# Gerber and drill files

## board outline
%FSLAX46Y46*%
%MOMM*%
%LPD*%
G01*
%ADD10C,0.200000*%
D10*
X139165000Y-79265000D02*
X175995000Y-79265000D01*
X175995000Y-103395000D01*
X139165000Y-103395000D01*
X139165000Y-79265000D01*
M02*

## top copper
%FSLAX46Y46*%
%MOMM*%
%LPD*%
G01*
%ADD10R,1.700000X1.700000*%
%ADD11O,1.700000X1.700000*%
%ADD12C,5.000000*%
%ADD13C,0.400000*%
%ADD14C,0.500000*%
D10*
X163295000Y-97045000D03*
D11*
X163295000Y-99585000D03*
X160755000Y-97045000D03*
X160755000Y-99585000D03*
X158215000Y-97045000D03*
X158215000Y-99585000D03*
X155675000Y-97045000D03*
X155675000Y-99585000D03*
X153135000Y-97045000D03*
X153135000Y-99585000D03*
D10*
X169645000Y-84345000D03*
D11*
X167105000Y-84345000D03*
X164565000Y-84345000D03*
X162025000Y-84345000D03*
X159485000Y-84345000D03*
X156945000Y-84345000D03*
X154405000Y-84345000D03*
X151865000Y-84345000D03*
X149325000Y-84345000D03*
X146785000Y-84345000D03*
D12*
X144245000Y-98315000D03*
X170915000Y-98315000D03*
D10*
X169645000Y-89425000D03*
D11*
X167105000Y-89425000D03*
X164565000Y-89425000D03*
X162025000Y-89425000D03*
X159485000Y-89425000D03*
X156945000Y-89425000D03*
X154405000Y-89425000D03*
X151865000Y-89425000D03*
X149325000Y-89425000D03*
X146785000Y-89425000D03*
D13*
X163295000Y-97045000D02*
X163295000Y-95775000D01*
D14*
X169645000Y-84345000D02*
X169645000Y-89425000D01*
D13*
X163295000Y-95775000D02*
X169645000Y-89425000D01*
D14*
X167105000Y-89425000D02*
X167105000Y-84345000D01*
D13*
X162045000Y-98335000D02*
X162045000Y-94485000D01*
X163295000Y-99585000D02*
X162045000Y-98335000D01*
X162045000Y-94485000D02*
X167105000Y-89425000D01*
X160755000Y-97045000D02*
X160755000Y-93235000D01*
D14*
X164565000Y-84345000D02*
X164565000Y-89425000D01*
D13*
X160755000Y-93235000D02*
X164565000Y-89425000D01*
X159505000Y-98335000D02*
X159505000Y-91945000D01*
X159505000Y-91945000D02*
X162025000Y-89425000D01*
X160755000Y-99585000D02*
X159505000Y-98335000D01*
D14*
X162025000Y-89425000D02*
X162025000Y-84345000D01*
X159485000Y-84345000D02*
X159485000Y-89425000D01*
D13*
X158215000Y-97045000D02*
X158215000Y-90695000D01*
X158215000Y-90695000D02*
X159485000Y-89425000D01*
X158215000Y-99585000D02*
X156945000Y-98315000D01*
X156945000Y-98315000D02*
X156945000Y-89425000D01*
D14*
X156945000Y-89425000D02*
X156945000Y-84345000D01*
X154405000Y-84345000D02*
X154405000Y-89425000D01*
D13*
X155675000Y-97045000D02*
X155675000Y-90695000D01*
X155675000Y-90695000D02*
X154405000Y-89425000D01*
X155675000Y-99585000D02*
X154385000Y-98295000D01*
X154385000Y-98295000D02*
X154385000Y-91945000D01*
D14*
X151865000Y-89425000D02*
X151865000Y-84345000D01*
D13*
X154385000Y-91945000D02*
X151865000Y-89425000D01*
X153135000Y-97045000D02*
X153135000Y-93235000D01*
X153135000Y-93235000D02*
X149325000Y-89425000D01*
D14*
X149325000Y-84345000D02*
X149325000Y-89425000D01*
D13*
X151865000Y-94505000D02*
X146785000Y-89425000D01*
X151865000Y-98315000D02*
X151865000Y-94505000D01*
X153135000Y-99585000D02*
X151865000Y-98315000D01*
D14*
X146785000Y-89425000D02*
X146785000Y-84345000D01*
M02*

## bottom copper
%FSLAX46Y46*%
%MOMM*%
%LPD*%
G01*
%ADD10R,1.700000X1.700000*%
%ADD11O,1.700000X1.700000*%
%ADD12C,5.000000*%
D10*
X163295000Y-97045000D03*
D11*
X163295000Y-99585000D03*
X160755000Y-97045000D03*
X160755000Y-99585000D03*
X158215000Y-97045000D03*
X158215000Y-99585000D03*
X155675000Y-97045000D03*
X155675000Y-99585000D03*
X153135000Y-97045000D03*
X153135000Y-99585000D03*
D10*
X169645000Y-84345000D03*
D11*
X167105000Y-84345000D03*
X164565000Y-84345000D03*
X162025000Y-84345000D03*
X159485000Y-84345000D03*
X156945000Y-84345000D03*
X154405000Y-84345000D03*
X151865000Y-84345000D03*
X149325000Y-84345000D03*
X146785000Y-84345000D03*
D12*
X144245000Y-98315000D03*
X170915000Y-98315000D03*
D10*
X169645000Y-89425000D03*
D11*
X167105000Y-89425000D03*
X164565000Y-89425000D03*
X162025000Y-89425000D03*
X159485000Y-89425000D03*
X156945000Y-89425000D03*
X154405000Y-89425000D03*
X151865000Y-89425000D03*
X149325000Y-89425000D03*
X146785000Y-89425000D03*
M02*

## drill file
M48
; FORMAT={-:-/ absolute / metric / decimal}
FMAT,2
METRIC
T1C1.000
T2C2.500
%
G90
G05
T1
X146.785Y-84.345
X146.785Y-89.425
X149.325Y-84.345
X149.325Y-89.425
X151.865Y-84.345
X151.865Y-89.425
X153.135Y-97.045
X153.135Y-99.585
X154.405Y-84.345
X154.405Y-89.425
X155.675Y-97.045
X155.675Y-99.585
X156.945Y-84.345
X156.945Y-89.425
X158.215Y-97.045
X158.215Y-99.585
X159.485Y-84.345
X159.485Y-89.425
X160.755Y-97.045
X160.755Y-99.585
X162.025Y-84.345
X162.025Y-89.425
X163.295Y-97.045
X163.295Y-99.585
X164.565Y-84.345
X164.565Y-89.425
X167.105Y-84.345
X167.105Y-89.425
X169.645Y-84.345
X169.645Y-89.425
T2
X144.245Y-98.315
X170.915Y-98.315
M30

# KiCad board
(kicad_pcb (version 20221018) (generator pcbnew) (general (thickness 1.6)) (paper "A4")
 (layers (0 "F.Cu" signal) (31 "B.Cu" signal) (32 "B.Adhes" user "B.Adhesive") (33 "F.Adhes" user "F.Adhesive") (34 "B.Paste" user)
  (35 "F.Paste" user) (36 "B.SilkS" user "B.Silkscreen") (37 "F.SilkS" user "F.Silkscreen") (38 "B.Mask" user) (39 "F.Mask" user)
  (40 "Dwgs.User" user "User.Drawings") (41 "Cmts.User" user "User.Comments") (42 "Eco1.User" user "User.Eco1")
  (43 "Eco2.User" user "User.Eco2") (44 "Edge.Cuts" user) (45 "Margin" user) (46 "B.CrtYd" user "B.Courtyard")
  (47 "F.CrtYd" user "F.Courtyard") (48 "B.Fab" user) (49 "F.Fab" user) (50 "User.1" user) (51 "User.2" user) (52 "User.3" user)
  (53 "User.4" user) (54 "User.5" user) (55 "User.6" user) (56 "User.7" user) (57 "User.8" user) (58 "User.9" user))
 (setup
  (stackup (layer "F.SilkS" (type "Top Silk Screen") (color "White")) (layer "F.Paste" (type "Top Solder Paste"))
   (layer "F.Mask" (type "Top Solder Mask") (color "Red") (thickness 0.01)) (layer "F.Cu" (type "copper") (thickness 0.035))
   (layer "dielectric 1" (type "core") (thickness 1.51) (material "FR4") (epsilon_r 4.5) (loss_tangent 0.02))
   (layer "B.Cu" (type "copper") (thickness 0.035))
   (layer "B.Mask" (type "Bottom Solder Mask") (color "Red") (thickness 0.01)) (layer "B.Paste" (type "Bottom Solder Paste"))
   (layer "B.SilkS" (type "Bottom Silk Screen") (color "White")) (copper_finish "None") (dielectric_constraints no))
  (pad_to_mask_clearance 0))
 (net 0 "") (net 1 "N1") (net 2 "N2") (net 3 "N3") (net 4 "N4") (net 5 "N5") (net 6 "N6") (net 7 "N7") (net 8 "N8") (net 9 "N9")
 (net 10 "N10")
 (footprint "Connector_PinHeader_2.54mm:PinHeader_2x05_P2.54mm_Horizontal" (layer "F.Cu") (at 163.295 97.045 -90)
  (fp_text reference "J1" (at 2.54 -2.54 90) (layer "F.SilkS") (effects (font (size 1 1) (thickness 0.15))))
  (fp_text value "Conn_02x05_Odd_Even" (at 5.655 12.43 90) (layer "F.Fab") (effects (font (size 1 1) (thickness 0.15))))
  (pad "1" thru_hole rect (at 0 0 270) (size 1.7 1.7) (drill 1) (layers "*.Cu" "*.Mask") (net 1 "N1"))
  (pad "2" thru_hole oval (at 2.54 0 270) (size 1.7 1.7) (drill 1) (layers "*.Cu" "*.Mask") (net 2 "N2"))
  (pad "3" thru_hole oval (at 0 2.54 270) (size 1.7 1.7) (drill 1) (layers "*.Cu" "*.Mask") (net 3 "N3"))
  (pad "4" thru_hole oval (at 2.54 2.54 270) (size 1.7 1.7) (drill 1) (layers "*.Cu" "*.Mask") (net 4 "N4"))
  (pad "5" thru_hole oval (at 0 5.08 270) (size 1.7 1.7) (drill 1) (layers "*.Cu" "*.Mask") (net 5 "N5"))
  (pad "6" thru_hole oval (at 2.54 5.08 270) (size 1.7 1.7) (drill 1) (layers "*.Cu" "*.Mask") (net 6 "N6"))
  (pad "7" thru_hole oval (at 0 7.62 270) (size 1.7 1.7) (drill 1) (layers "*.Cu" "*.Mask") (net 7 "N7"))
  (pad "8" thru_hole oval (at 2.54 7.62 270) (size 1.7 1.7) (drill 1) (layers "*.Cu" "*.Mask") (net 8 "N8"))
  (pad "9" thru_hole oval (at 0 10.16 270) (size 1.7 1.7) (drill 1) (layers "*.Cu" "*.Mask") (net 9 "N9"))
  (pad "10" thru_hole oval (at 2.54 10.16 270) (size 1.7 1.7) (drill 1) (layers "*.Cu" "*.Mask") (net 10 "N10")))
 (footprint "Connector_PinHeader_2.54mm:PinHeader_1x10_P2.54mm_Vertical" (layer "F.Cu") (at 169.645 84.345 -90)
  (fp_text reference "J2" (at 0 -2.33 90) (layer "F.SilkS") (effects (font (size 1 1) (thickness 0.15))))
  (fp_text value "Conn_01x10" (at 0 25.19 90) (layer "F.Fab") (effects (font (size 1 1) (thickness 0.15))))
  (pad "1" thru_hole rect (at 0 0 270) (size 1.7 1.7) (drill 1) (layers "*.Cu" "*.Mask") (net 1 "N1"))
  (pad "2" thru_hole oval (at 0 2.54 270) (size 1.7 1.7) (drill 1) (layers "*.Cu" "*.Mask") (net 2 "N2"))
  (pad "3" thru_hole oval (at 0 5.08 270) (size 1.7 1.7) (drill 1) (layers "*.Cu" "*.Mask") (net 3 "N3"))
  (pad "4" thru_hole oval (at 0 7.62 270) (size 1.7 1.7) (drill 1) (layers "*.Cu" "*.Mask") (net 4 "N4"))
  (pad "5" thru_hole oval (at 0 10.16 270) (size 1.7 1.7) (drill 1) (layers "*.Cu" "*.Mask") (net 5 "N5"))
  (pad "6" thru_hole oval (at 0 12.7 270) (size 1.7 1.7) (drill 1) (layers "*.Cu" "*.Mask") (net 6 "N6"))
  (pad "7" thru_hole oval (at 0 15.24 270) (size 1.7 1.7) (drill 1) (layers "*.Cu" "*.Mask") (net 7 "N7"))
  (pad "8" thru_hole oval (at 0 17.78 270) (size 1.7 1.7) (drill 1) (layers "*.Cu" "*.Mask") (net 8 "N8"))
  (pad "9" thru_hole oval (at 0 20.32 270) (size 1.7 1.7) (drill 1) (layers "*.Cu" "*.Mask") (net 9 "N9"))
  (pad "10" thru_hole oval (at 0 22.86 270) (size 1.7 1.7) (drill 1) (layers "*.Cu" "*.Mask") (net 10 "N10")))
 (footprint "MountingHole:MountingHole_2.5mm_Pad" (layer "F.Cu") (at 144.245 98.315 -90)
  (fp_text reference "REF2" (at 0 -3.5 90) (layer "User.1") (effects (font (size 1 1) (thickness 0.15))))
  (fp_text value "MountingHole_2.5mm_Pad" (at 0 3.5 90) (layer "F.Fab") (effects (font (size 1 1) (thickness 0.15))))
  (pad "2" thru_hole circle (at 0 0 270) (size 5 5) (drill 2.5) (layers "*.Cu" "*.Mask")))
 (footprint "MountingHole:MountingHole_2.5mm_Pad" (layer "F.Cu") (at 170.915 98.315 -90)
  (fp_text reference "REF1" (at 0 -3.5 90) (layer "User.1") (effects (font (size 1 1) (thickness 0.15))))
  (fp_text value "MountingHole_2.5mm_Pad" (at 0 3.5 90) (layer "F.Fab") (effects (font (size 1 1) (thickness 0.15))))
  (pad "1" thru_hole circle (at 0 0 270) (size 5 5) (drill 2.5) (layers "*.Cu" "*.Mask")))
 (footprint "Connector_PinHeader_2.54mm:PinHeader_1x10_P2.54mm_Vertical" (layer "F.Cu") (at 169.645 89.425 -90)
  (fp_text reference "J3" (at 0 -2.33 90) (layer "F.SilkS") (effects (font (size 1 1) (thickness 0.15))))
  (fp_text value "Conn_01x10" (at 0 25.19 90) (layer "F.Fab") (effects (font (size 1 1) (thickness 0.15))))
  (pad "1" thru_hole rect (at 0 0 270) (size 1.7 1.7) (drill 1) (layers "*.Cu" "*.Mask") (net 1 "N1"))
  (pad "2" thru_hole oval (at 0 2.54 270) (size 1.7 1.7) (drill 1) (layers "*.Cu" "*.Mask") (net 2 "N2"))
  (pad "3" thru_hole oval (at 0 5.08 270) (size 1.7 1.7) (drill 1) (layers "*.Cu" "*.Mask") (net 3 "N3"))
  (pad "4" thru_hole oval (at 0 7.62 270) (size 1.7 1.7) (drill 1) (layers "*.Cu" "*.Mask") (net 4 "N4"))
  (pad "5" thru_hole oval (at 0 10.16 270) (size 1.7 1.7) (drill 1) (layers "*.Cu" "*.Mask") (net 5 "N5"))
  (pad "6" thru_hole oval (at 0 12.7 270) (size 1.7 1.7) (drill 1) (layers "*.Cu" "*.Mask") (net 6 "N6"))
  (pad "7" thru_hole oval (at 0 15.24 270) (size 1.7 1.7) (drill 1) (layers "*.Cu" "*.Mask") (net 7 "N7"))
  (pad "8" thru_hole oval (at 0 17.78 270) (size 1.7 1.7) (drill 1) (layers "*.Cu" "*.Mask") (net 8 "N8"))
  (pad "9" thru_hole oval (at 0 20.32 270) (size 1.7 1.7) (drill 1) (layers "*.Cu" "*.Mask") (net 9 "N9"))
  (pad "10" thru_hole oval (at 0 22.86 270) (size 1.7 1.7) (drill 1) (layers "*.Cu" "*.Mask") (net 10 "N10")))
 (gr_rect (start 175.995 79.265) (end 139.165 103.395) (stroke (width 0.2) (type default)) (fill none) (layer "Edge.Cuts"))
 (segment (start 163.295 97.045) (end 163.295 95.775) (width 0.4) (layer "F.Cu") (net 1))
 (segment (start 169.645 84.345) (end 169.645 89.425) (width 0.5) (layer "F.Cu") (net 1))
 (segment (start 163.295 95.775) (end 169.645 89.425) (width 0.4) (layer "F.Cu") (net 1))
 (segment (start 167.105 89.425) (end 167.105 84.345) (width 0.5) (layer "F.Cu") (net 2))
 (segment (start 162.045 98.335) (end 162.045 94.485) (width 0.4) (layer "F.Cu") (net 2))
 (segment (start 163.295 99.585) (end 162.045 98.335) (width 0.4) (layer "F.Cu") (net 2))
 (segment (start 162.045 94.485) (end 167.105 89.425) (width 0.4) (layer "F.Cu") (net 2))
 (segment (start 160.755 97.045) (end 160.755 93.235) (width 0.4) (layer "F.Cu") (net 3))
 (segment (start 164.565 84.345) (end 164.565 89.425) (width 0.5) (layer "F.Cu") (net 3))
 (segment (start 160.755 93.235) (end 164.565 89.425) (width 0.4) (layer "F.Cu") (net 3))
 (segment (start 159.505 98.335) (end 159.505 91.945) (width 0.4) (layer "F.Cu") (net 4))
 (segment (start 159.505 91.945) (end 162.025 89.425) (width 0.4) (layer "F.Cu") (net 4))
 (segment (start 160.755 99.585) (end 159.505 98.335) (width 0.4) (layer "F.Cu") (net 4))
 (segment (start 162.025 89.425) (end 162.025 84.345) (width 0.5) (layer "F.Cu") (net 4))
 (segment (start 159.485 84.345) (end 159.485 89.425) (width 0.5) (layer "F.Cu") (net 5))
 (segment (start 158.215 97.045) (end 158.215 90.695) (width 0.4) (layer "F.Cu") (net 5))
 (segment (start 158.215 90.695) (end 159.485 89.425) (width 0.4) (layer "F.Cu") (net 5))
 (segment (start 158.215 99.585) (end 156.945 98.315) (width 0.4) (layer "F.Cu") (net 6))
 (segment (start 156.945 98.315) (end 156.945 89.425) (width 0.4) (layer "F.Cu") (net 6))
 (segment (start 156.945 89.425) (end 156.945 84.345) (width 0.5) (layer "F.Cu") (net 6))
 (segment (start 154.405 84.345) (end 154.405 89.425) (width 0.5) (layer "F.Cu") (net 7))
 (segment (start 155.675 97.045) (end 155.675 90.695) (width 0.4) (layer "F.Cu") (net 7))
 (segment (start 155.675 90.695) (end 154.405 89.425) (width 0.4) (layer "F.Cu") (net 7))
 (segment (start 155.675 99.585) (end 154.385 98.295) (width 0.4) (layer "F.Cu") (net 8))
 (segment (start 154.385 98.295) (end 154.385 91.945) (width 0.4) (layer "F.Cu") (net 8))
 (segment (start 151.865 89.425) (end 151.865 84.345) (width 0.5) (layer "F.Cu") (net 8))
 (segment (start 154.385 91.945) (end 151.865 89.425) (width 0.4) (layer "F.Cu") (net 8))
 (segment (start 153.135 97.045) (end 153.135 93.235) (width 0.4) (layer "F.Cu") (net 9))
 (segment (start 153.135 93.235) (end 149.325 89.425) (width 0.4) (layer "F.Cu") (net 9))
 (segment (start 149.325 84.345) (end 149.325 89.425) (width 0.5) (layer "F.Cu") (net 9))
 (segment (start 151.865 94.505) (end 146.785 89.425) (width 0.4) (layer "F.Cu") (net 10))
 (segment (start 151.865 98.315) (end 151.865 94.505) (width 0.4) (layer "F.Cu") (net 10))
 (segment (start 153.135 99.585) (end 151.865 98.315) (width 0.4) (layer "F.Cu") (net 10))
 (segment (start 146.785 89.425) (end 146.785 84.345) (width 0.5) (layer "F.Cu") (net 10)))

